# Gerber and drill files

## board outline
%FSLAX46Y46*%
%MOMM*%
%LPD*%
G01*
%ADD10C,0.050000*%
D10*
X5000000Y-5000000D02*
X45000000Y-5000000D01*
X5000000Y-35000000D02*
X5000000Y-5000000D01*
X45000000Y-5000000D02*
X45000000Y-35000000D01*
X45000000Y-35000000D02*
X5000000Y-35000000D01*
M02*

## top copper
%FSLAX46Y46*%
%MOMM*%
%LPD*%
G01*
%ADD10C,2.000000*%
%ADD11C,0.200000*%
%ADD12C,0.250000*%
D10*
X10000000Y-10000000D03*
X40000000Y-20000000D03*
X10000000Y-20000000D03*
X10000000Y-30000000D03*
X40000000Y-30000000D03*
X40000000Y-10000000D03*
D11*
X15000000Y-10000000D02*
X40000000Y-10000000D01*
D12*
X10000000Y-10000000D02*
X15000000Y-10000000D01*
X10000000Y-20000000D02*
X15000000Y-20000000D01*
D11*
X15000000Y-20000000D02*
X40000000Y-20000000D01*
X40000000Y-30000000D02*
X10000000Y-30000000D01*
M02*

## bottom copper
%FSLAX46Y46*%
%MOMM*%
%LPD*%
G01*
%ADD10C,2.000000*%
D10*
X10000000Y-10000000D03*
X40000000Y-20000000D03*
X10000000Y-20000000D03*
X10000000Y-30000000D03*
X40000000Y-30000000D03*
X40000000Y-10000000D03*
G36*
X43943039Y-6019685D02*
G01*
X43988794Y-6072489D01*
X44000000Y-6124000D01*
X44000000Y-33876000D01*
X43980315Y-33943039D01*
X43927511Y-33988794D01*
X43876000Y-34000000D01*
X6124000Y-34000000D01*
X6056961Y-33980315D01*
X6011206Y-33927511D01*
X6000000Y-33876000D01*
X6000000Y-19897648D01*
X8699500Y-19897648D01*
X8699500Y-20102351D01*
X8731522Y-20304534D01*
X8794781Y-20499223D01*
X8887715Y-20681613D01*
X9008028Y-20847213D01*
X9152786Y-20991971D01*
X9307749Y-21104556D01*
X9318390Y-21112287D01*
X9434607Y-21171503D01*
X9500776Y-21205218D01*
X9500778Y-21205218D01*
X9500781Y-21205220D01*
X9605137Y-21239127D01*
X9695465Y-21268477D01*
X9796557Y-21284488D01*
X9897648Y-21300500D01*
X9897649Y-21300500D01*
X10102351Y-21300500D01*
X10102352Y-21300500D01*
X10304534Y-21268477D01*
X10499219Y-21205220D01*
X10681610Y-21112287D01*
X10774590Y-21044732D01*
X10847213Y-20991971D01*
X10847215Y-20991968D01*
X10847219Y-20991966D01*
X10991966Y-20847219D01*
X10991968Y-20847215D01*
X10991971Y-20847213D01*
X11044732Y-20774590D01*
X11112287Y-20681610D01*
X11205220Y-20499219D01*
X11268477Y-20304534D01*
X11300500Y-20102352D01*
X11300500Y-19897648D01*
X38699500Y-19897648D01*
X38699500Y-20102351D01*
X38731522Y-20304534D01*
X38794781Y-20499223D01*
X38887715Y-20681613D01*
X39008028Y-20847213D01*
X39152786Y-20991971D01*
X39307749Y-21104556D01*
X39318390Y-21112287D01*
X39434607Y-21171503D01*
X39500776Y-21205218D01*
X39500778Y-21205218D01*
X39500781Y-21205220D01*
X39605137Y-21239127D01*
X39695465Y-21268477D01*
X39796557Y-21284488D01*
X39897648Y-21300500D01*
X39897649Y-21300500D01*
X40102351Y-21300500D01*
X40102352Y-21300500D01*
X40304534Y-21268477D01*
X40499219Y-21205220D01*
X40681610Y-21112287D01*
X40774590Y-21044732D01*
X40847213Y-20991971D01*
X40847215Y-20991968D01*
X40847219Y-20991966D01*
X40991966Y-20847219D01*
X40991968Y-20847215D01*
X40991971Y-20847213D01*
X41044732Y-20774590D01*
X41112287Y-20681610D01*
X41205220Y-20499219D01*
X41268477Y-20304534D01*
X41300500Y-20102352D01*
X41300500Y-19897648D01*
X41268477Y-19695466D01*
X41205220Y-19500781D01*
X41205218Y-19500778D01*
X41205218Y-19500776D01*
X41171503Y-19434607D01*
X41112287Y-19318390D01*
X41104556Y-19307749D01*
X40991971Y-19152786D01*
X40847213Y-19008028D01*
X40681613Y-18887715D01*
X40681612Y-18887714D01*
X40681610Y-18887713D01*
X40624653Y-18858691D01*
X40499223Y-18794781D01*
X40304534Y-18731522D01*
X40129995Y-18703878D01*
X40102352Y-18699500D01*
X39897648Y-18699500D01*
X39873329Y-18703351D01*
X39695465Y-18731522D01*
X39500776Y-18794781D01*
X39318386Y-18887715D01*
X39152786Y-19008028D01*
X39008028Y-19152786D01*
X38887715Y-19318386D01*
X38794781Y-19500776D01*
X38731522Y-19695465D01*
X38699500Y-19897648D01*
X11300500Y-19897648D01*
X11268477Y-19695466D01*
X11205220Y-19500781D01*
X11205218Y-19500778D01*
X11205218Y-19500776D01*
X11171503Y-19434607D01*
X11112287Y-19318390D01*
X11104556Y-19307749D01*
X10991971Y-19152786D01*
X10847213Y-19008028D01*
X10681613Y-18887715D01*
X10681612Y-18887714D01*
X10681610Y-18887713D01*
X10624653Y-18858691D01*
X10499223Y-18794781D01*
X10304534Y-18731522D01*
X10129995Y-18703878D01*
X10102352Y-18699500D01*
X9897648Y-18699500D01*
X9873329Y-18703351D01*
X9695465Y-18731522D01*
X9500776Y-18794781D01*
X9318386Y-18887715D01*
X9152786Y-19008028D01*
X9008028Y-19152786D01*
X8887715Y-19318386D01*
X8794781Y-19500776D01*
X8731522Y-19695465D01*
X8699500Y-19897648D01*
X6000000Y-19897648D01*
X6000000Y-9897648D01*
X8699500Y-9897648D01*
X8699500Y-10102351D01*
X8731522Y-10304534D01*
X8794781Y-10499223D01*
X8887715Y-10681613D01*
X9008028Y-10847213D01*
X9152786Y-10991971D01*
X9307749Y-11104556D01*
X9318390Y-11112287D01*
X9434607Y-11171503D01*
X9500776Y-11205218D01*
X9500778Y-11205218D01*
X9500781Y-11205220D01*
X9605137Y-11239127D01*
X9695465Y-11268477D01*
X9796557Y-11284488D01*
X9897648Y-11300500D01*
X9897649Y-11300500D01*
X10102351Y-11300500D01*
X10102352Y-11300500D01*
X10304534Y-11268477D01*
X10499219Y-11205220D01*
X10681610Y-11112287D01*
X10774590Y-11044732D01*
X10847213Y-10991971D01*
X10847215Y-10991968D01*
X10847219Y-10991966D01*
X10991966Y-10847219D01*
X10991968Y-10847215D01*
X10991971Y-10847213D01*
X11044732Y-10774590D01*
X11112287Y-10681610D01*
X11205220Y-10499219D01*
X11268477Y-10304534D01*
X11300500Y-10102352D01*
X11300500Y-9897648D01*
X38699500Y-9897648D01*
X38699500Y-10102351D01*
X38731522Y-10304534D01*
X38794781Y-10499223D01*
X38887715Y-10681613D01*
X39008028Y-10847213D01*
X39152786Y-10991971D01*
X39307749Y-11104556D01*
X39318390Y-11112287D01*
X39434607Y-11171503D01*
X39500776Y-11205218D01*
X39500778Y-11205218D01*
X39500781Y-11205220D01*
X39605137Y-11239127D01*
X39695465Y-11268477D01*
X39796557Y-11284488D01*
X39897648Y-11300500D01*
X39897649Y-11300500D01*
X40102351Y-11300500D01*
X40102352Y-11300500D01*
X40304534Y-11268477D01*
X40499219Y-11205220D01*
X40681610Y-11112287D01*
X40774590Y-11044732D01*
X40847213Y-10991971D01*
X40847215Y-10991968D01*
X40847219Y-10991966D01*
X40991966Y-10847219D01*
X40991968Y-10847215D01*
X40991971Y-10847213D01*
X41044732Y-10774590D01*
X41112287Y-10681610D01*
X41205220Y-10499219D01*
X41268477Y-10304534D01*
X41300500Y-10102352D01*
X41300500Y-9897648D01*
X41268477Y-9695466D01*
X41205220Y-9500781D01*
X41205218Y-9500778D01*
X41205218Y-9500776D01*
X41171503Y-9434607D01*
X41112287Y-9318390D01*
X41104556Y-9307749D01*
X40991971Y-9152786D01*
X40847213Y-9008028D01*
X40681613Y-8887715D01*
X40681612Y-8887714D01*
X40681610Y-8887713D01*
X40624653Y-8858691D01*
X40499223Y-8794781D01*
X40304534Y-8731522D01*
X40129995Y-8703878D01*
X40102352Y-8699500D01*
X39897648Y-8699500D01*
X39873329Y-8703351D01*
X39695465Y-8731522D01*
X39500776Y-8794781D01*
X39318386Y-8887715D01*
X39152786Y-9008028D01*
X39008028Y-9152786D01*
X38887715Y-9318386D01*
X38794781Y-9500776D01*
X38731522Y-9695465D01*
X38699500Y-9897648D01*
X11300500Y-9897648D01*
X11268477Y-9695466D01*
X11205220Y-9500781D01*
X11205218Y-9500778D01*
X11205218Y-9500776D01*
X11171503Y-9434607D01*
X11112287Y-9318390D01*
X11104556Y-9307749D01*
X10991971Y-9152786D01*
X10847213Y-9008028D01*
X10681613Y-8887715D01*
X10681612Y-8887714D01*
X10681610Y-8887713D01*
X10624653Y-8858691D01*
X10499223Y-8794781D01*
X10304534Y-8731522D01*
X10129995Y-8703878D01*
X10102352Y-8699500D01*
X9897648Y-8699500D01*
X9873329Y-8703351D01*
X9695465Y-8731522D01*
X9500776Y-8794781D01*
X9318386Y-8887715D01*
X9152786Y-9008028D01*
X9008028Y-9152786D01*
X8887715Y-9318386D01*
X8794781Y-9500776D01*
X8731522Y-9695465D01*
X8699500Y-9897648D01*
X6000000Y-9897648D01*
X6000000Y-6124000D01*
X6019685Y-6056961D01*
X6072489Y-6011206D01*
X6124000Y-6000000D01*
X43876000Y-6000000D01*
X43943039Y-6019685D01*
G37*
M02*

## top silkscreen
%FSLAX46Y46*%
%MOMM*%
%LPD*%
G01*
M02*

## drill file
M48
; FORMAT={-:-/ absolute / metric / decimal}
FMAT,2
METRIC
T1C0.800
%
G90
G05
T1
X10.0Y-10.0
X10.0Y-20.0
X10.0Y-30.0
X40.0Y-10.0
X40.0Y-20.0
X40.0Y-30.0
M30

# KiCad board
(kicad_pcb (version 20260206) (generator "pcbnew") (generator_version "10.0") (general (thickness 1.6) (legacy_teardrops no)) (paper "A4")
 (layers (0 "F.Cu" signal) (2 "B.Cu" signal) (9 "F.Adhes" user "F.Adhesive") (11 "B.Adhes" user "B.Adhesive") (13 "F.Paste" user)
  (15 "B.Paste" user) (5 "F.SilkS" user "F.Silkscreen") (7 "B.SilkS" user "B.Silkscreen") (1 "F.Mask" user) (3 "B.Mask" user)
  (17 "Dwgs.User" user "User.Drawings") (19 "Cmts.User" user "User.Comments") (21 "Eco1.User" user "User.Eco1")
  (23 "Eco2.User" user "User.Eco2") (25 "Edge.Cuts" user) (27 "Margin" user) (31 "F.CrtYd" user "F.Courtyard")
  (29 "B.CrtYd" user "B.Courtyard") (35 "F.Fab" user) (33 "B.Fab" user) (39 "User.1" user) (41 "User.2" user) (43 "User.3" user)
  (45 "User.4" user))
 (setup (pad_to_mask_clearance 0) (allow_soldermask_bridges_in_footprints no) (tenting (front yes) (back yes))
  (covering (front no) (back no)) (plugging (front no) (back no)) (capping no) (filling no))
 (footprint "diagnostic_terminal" (layer "F.Cu") (at 10 10)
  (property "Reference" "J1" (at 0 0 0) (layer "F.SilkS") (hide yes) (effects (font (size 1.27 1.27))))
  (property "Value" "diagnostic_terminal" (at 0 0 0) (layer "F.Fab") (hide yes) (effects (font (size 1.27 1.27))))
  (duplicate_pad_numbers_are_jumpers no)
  (pad "1" thru_hole circle (at 0 0) (size 2 2) (drill 0.8) (layers "*.Cu") (remove_unused_layers no) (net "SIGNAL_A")))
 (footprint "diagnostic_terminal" (layer "F.Cu") (at 40 20)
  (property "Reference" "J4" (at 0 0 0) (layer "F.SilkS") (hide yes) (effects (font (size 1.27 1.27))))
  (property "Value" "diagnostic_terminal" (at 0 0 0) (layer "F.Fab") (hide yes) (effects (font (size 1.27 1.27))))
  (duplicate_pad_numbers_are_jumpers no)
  (pad "1" thru_hole circle (at 0 0) (size 2 2) (drill 0.8) (layers "*.Cu") (remove_unused_layers no) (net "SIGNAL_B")))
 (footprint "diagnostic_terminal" (layer "F.Cu") (at 10 20)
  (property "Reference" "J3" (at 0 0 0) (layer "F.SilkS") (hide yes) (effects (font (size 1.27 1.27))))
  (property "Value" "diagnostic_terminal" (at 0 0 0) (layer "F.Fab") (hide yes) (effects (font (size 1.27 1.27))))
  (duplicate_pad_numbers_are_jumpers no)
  (pad "1" thru_hole circle (at 0 0) (size 2 2) (drill 0.8) (layers "*.Cu") (remove_unused_layers no) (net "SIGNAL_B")))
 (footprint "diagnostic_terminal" (layer "F.Cu") (at 10 30)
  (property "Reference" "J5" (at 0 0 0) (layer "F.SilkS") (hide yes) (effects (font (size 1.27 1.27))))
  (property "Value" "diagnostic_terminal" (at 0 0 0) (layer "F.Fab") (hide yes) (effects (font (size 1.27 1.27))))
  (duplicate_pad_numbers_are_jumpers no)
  (pad "1" thru_hole circle (at 0 0) (size 2 2) (drill 0.8) (layers "*.Cu") (remove_unused_layers no) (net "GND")))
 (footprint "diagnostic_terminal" (layer "F.Cu") (at 40 30)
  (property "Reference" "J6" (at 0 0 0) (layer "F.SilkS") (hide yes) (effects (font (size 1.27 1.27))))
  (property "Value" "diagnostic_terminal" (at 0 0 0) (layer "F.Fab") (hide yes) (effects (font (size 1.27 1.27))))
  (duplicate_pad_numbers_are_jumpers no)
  (pad "1" thru_hole circle (at 0 0) (size 2 2) (drill 0.8) (layers "*.Cu") (remove_unused_layers no) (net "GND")))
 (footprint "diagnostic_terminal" (layer "F.Cu") (at 40 10)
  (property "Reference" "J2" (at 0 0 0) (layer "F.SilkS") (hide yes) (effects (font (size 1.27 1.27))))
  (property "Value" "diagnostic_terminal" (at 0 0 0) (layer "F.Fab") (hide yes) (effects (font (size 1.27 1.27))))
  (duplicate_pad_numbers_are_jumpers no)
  (pad "1" thru_hole circle (at 0 0) (size 2 2) (drill 0.8) (layers "*.Cu") (remove_unused_layers no) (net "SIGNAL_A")))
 (gr_line (start 5 5) (end 45 5) (stroke (width 0.05) (type default)) (layer "Edge.Cuts"))
 (gr_line (start 5 35) (end 5 5) (stroke (width 0.05) (type default)) (layer "Edge.Cuts"))
 (gr_line (start 45 5) (end 45 35) (stroke (width 0.05) (type default)) (layer "Edge.Cuts"))
 (gr_line (start 45 35) (end 5 35) (stroke (width 0.05) (type default)) (layer "Edge.Cuts"))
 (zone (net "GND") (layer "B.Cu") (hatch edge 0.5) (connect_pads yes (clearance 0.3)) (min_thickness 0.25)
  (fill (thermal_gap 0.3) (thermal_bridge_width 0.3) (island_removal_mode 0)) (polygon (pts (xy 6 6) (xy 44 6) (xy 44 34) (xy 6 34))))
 (segment (start 15 10) (end 40 10) (width 0.2) (layer "F.Cu") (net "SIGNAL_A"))
 (segment (locked yes) (start 10 10) (end 15 10) (width 0.25) (layer "F.Cu") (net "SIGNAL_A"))
 (segment (locked yes) (start 10 20) (end 15 20) (width 0.25) (layer "F.Cu") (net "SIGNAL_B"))
 (segment (start 15 20) (end 40 20) (width 0.2) (layer "F.Cu") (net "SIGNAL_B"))
 (segment (start 40 30) (end 10 30) (width 0.2) (layer "F.Cu") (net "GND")))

